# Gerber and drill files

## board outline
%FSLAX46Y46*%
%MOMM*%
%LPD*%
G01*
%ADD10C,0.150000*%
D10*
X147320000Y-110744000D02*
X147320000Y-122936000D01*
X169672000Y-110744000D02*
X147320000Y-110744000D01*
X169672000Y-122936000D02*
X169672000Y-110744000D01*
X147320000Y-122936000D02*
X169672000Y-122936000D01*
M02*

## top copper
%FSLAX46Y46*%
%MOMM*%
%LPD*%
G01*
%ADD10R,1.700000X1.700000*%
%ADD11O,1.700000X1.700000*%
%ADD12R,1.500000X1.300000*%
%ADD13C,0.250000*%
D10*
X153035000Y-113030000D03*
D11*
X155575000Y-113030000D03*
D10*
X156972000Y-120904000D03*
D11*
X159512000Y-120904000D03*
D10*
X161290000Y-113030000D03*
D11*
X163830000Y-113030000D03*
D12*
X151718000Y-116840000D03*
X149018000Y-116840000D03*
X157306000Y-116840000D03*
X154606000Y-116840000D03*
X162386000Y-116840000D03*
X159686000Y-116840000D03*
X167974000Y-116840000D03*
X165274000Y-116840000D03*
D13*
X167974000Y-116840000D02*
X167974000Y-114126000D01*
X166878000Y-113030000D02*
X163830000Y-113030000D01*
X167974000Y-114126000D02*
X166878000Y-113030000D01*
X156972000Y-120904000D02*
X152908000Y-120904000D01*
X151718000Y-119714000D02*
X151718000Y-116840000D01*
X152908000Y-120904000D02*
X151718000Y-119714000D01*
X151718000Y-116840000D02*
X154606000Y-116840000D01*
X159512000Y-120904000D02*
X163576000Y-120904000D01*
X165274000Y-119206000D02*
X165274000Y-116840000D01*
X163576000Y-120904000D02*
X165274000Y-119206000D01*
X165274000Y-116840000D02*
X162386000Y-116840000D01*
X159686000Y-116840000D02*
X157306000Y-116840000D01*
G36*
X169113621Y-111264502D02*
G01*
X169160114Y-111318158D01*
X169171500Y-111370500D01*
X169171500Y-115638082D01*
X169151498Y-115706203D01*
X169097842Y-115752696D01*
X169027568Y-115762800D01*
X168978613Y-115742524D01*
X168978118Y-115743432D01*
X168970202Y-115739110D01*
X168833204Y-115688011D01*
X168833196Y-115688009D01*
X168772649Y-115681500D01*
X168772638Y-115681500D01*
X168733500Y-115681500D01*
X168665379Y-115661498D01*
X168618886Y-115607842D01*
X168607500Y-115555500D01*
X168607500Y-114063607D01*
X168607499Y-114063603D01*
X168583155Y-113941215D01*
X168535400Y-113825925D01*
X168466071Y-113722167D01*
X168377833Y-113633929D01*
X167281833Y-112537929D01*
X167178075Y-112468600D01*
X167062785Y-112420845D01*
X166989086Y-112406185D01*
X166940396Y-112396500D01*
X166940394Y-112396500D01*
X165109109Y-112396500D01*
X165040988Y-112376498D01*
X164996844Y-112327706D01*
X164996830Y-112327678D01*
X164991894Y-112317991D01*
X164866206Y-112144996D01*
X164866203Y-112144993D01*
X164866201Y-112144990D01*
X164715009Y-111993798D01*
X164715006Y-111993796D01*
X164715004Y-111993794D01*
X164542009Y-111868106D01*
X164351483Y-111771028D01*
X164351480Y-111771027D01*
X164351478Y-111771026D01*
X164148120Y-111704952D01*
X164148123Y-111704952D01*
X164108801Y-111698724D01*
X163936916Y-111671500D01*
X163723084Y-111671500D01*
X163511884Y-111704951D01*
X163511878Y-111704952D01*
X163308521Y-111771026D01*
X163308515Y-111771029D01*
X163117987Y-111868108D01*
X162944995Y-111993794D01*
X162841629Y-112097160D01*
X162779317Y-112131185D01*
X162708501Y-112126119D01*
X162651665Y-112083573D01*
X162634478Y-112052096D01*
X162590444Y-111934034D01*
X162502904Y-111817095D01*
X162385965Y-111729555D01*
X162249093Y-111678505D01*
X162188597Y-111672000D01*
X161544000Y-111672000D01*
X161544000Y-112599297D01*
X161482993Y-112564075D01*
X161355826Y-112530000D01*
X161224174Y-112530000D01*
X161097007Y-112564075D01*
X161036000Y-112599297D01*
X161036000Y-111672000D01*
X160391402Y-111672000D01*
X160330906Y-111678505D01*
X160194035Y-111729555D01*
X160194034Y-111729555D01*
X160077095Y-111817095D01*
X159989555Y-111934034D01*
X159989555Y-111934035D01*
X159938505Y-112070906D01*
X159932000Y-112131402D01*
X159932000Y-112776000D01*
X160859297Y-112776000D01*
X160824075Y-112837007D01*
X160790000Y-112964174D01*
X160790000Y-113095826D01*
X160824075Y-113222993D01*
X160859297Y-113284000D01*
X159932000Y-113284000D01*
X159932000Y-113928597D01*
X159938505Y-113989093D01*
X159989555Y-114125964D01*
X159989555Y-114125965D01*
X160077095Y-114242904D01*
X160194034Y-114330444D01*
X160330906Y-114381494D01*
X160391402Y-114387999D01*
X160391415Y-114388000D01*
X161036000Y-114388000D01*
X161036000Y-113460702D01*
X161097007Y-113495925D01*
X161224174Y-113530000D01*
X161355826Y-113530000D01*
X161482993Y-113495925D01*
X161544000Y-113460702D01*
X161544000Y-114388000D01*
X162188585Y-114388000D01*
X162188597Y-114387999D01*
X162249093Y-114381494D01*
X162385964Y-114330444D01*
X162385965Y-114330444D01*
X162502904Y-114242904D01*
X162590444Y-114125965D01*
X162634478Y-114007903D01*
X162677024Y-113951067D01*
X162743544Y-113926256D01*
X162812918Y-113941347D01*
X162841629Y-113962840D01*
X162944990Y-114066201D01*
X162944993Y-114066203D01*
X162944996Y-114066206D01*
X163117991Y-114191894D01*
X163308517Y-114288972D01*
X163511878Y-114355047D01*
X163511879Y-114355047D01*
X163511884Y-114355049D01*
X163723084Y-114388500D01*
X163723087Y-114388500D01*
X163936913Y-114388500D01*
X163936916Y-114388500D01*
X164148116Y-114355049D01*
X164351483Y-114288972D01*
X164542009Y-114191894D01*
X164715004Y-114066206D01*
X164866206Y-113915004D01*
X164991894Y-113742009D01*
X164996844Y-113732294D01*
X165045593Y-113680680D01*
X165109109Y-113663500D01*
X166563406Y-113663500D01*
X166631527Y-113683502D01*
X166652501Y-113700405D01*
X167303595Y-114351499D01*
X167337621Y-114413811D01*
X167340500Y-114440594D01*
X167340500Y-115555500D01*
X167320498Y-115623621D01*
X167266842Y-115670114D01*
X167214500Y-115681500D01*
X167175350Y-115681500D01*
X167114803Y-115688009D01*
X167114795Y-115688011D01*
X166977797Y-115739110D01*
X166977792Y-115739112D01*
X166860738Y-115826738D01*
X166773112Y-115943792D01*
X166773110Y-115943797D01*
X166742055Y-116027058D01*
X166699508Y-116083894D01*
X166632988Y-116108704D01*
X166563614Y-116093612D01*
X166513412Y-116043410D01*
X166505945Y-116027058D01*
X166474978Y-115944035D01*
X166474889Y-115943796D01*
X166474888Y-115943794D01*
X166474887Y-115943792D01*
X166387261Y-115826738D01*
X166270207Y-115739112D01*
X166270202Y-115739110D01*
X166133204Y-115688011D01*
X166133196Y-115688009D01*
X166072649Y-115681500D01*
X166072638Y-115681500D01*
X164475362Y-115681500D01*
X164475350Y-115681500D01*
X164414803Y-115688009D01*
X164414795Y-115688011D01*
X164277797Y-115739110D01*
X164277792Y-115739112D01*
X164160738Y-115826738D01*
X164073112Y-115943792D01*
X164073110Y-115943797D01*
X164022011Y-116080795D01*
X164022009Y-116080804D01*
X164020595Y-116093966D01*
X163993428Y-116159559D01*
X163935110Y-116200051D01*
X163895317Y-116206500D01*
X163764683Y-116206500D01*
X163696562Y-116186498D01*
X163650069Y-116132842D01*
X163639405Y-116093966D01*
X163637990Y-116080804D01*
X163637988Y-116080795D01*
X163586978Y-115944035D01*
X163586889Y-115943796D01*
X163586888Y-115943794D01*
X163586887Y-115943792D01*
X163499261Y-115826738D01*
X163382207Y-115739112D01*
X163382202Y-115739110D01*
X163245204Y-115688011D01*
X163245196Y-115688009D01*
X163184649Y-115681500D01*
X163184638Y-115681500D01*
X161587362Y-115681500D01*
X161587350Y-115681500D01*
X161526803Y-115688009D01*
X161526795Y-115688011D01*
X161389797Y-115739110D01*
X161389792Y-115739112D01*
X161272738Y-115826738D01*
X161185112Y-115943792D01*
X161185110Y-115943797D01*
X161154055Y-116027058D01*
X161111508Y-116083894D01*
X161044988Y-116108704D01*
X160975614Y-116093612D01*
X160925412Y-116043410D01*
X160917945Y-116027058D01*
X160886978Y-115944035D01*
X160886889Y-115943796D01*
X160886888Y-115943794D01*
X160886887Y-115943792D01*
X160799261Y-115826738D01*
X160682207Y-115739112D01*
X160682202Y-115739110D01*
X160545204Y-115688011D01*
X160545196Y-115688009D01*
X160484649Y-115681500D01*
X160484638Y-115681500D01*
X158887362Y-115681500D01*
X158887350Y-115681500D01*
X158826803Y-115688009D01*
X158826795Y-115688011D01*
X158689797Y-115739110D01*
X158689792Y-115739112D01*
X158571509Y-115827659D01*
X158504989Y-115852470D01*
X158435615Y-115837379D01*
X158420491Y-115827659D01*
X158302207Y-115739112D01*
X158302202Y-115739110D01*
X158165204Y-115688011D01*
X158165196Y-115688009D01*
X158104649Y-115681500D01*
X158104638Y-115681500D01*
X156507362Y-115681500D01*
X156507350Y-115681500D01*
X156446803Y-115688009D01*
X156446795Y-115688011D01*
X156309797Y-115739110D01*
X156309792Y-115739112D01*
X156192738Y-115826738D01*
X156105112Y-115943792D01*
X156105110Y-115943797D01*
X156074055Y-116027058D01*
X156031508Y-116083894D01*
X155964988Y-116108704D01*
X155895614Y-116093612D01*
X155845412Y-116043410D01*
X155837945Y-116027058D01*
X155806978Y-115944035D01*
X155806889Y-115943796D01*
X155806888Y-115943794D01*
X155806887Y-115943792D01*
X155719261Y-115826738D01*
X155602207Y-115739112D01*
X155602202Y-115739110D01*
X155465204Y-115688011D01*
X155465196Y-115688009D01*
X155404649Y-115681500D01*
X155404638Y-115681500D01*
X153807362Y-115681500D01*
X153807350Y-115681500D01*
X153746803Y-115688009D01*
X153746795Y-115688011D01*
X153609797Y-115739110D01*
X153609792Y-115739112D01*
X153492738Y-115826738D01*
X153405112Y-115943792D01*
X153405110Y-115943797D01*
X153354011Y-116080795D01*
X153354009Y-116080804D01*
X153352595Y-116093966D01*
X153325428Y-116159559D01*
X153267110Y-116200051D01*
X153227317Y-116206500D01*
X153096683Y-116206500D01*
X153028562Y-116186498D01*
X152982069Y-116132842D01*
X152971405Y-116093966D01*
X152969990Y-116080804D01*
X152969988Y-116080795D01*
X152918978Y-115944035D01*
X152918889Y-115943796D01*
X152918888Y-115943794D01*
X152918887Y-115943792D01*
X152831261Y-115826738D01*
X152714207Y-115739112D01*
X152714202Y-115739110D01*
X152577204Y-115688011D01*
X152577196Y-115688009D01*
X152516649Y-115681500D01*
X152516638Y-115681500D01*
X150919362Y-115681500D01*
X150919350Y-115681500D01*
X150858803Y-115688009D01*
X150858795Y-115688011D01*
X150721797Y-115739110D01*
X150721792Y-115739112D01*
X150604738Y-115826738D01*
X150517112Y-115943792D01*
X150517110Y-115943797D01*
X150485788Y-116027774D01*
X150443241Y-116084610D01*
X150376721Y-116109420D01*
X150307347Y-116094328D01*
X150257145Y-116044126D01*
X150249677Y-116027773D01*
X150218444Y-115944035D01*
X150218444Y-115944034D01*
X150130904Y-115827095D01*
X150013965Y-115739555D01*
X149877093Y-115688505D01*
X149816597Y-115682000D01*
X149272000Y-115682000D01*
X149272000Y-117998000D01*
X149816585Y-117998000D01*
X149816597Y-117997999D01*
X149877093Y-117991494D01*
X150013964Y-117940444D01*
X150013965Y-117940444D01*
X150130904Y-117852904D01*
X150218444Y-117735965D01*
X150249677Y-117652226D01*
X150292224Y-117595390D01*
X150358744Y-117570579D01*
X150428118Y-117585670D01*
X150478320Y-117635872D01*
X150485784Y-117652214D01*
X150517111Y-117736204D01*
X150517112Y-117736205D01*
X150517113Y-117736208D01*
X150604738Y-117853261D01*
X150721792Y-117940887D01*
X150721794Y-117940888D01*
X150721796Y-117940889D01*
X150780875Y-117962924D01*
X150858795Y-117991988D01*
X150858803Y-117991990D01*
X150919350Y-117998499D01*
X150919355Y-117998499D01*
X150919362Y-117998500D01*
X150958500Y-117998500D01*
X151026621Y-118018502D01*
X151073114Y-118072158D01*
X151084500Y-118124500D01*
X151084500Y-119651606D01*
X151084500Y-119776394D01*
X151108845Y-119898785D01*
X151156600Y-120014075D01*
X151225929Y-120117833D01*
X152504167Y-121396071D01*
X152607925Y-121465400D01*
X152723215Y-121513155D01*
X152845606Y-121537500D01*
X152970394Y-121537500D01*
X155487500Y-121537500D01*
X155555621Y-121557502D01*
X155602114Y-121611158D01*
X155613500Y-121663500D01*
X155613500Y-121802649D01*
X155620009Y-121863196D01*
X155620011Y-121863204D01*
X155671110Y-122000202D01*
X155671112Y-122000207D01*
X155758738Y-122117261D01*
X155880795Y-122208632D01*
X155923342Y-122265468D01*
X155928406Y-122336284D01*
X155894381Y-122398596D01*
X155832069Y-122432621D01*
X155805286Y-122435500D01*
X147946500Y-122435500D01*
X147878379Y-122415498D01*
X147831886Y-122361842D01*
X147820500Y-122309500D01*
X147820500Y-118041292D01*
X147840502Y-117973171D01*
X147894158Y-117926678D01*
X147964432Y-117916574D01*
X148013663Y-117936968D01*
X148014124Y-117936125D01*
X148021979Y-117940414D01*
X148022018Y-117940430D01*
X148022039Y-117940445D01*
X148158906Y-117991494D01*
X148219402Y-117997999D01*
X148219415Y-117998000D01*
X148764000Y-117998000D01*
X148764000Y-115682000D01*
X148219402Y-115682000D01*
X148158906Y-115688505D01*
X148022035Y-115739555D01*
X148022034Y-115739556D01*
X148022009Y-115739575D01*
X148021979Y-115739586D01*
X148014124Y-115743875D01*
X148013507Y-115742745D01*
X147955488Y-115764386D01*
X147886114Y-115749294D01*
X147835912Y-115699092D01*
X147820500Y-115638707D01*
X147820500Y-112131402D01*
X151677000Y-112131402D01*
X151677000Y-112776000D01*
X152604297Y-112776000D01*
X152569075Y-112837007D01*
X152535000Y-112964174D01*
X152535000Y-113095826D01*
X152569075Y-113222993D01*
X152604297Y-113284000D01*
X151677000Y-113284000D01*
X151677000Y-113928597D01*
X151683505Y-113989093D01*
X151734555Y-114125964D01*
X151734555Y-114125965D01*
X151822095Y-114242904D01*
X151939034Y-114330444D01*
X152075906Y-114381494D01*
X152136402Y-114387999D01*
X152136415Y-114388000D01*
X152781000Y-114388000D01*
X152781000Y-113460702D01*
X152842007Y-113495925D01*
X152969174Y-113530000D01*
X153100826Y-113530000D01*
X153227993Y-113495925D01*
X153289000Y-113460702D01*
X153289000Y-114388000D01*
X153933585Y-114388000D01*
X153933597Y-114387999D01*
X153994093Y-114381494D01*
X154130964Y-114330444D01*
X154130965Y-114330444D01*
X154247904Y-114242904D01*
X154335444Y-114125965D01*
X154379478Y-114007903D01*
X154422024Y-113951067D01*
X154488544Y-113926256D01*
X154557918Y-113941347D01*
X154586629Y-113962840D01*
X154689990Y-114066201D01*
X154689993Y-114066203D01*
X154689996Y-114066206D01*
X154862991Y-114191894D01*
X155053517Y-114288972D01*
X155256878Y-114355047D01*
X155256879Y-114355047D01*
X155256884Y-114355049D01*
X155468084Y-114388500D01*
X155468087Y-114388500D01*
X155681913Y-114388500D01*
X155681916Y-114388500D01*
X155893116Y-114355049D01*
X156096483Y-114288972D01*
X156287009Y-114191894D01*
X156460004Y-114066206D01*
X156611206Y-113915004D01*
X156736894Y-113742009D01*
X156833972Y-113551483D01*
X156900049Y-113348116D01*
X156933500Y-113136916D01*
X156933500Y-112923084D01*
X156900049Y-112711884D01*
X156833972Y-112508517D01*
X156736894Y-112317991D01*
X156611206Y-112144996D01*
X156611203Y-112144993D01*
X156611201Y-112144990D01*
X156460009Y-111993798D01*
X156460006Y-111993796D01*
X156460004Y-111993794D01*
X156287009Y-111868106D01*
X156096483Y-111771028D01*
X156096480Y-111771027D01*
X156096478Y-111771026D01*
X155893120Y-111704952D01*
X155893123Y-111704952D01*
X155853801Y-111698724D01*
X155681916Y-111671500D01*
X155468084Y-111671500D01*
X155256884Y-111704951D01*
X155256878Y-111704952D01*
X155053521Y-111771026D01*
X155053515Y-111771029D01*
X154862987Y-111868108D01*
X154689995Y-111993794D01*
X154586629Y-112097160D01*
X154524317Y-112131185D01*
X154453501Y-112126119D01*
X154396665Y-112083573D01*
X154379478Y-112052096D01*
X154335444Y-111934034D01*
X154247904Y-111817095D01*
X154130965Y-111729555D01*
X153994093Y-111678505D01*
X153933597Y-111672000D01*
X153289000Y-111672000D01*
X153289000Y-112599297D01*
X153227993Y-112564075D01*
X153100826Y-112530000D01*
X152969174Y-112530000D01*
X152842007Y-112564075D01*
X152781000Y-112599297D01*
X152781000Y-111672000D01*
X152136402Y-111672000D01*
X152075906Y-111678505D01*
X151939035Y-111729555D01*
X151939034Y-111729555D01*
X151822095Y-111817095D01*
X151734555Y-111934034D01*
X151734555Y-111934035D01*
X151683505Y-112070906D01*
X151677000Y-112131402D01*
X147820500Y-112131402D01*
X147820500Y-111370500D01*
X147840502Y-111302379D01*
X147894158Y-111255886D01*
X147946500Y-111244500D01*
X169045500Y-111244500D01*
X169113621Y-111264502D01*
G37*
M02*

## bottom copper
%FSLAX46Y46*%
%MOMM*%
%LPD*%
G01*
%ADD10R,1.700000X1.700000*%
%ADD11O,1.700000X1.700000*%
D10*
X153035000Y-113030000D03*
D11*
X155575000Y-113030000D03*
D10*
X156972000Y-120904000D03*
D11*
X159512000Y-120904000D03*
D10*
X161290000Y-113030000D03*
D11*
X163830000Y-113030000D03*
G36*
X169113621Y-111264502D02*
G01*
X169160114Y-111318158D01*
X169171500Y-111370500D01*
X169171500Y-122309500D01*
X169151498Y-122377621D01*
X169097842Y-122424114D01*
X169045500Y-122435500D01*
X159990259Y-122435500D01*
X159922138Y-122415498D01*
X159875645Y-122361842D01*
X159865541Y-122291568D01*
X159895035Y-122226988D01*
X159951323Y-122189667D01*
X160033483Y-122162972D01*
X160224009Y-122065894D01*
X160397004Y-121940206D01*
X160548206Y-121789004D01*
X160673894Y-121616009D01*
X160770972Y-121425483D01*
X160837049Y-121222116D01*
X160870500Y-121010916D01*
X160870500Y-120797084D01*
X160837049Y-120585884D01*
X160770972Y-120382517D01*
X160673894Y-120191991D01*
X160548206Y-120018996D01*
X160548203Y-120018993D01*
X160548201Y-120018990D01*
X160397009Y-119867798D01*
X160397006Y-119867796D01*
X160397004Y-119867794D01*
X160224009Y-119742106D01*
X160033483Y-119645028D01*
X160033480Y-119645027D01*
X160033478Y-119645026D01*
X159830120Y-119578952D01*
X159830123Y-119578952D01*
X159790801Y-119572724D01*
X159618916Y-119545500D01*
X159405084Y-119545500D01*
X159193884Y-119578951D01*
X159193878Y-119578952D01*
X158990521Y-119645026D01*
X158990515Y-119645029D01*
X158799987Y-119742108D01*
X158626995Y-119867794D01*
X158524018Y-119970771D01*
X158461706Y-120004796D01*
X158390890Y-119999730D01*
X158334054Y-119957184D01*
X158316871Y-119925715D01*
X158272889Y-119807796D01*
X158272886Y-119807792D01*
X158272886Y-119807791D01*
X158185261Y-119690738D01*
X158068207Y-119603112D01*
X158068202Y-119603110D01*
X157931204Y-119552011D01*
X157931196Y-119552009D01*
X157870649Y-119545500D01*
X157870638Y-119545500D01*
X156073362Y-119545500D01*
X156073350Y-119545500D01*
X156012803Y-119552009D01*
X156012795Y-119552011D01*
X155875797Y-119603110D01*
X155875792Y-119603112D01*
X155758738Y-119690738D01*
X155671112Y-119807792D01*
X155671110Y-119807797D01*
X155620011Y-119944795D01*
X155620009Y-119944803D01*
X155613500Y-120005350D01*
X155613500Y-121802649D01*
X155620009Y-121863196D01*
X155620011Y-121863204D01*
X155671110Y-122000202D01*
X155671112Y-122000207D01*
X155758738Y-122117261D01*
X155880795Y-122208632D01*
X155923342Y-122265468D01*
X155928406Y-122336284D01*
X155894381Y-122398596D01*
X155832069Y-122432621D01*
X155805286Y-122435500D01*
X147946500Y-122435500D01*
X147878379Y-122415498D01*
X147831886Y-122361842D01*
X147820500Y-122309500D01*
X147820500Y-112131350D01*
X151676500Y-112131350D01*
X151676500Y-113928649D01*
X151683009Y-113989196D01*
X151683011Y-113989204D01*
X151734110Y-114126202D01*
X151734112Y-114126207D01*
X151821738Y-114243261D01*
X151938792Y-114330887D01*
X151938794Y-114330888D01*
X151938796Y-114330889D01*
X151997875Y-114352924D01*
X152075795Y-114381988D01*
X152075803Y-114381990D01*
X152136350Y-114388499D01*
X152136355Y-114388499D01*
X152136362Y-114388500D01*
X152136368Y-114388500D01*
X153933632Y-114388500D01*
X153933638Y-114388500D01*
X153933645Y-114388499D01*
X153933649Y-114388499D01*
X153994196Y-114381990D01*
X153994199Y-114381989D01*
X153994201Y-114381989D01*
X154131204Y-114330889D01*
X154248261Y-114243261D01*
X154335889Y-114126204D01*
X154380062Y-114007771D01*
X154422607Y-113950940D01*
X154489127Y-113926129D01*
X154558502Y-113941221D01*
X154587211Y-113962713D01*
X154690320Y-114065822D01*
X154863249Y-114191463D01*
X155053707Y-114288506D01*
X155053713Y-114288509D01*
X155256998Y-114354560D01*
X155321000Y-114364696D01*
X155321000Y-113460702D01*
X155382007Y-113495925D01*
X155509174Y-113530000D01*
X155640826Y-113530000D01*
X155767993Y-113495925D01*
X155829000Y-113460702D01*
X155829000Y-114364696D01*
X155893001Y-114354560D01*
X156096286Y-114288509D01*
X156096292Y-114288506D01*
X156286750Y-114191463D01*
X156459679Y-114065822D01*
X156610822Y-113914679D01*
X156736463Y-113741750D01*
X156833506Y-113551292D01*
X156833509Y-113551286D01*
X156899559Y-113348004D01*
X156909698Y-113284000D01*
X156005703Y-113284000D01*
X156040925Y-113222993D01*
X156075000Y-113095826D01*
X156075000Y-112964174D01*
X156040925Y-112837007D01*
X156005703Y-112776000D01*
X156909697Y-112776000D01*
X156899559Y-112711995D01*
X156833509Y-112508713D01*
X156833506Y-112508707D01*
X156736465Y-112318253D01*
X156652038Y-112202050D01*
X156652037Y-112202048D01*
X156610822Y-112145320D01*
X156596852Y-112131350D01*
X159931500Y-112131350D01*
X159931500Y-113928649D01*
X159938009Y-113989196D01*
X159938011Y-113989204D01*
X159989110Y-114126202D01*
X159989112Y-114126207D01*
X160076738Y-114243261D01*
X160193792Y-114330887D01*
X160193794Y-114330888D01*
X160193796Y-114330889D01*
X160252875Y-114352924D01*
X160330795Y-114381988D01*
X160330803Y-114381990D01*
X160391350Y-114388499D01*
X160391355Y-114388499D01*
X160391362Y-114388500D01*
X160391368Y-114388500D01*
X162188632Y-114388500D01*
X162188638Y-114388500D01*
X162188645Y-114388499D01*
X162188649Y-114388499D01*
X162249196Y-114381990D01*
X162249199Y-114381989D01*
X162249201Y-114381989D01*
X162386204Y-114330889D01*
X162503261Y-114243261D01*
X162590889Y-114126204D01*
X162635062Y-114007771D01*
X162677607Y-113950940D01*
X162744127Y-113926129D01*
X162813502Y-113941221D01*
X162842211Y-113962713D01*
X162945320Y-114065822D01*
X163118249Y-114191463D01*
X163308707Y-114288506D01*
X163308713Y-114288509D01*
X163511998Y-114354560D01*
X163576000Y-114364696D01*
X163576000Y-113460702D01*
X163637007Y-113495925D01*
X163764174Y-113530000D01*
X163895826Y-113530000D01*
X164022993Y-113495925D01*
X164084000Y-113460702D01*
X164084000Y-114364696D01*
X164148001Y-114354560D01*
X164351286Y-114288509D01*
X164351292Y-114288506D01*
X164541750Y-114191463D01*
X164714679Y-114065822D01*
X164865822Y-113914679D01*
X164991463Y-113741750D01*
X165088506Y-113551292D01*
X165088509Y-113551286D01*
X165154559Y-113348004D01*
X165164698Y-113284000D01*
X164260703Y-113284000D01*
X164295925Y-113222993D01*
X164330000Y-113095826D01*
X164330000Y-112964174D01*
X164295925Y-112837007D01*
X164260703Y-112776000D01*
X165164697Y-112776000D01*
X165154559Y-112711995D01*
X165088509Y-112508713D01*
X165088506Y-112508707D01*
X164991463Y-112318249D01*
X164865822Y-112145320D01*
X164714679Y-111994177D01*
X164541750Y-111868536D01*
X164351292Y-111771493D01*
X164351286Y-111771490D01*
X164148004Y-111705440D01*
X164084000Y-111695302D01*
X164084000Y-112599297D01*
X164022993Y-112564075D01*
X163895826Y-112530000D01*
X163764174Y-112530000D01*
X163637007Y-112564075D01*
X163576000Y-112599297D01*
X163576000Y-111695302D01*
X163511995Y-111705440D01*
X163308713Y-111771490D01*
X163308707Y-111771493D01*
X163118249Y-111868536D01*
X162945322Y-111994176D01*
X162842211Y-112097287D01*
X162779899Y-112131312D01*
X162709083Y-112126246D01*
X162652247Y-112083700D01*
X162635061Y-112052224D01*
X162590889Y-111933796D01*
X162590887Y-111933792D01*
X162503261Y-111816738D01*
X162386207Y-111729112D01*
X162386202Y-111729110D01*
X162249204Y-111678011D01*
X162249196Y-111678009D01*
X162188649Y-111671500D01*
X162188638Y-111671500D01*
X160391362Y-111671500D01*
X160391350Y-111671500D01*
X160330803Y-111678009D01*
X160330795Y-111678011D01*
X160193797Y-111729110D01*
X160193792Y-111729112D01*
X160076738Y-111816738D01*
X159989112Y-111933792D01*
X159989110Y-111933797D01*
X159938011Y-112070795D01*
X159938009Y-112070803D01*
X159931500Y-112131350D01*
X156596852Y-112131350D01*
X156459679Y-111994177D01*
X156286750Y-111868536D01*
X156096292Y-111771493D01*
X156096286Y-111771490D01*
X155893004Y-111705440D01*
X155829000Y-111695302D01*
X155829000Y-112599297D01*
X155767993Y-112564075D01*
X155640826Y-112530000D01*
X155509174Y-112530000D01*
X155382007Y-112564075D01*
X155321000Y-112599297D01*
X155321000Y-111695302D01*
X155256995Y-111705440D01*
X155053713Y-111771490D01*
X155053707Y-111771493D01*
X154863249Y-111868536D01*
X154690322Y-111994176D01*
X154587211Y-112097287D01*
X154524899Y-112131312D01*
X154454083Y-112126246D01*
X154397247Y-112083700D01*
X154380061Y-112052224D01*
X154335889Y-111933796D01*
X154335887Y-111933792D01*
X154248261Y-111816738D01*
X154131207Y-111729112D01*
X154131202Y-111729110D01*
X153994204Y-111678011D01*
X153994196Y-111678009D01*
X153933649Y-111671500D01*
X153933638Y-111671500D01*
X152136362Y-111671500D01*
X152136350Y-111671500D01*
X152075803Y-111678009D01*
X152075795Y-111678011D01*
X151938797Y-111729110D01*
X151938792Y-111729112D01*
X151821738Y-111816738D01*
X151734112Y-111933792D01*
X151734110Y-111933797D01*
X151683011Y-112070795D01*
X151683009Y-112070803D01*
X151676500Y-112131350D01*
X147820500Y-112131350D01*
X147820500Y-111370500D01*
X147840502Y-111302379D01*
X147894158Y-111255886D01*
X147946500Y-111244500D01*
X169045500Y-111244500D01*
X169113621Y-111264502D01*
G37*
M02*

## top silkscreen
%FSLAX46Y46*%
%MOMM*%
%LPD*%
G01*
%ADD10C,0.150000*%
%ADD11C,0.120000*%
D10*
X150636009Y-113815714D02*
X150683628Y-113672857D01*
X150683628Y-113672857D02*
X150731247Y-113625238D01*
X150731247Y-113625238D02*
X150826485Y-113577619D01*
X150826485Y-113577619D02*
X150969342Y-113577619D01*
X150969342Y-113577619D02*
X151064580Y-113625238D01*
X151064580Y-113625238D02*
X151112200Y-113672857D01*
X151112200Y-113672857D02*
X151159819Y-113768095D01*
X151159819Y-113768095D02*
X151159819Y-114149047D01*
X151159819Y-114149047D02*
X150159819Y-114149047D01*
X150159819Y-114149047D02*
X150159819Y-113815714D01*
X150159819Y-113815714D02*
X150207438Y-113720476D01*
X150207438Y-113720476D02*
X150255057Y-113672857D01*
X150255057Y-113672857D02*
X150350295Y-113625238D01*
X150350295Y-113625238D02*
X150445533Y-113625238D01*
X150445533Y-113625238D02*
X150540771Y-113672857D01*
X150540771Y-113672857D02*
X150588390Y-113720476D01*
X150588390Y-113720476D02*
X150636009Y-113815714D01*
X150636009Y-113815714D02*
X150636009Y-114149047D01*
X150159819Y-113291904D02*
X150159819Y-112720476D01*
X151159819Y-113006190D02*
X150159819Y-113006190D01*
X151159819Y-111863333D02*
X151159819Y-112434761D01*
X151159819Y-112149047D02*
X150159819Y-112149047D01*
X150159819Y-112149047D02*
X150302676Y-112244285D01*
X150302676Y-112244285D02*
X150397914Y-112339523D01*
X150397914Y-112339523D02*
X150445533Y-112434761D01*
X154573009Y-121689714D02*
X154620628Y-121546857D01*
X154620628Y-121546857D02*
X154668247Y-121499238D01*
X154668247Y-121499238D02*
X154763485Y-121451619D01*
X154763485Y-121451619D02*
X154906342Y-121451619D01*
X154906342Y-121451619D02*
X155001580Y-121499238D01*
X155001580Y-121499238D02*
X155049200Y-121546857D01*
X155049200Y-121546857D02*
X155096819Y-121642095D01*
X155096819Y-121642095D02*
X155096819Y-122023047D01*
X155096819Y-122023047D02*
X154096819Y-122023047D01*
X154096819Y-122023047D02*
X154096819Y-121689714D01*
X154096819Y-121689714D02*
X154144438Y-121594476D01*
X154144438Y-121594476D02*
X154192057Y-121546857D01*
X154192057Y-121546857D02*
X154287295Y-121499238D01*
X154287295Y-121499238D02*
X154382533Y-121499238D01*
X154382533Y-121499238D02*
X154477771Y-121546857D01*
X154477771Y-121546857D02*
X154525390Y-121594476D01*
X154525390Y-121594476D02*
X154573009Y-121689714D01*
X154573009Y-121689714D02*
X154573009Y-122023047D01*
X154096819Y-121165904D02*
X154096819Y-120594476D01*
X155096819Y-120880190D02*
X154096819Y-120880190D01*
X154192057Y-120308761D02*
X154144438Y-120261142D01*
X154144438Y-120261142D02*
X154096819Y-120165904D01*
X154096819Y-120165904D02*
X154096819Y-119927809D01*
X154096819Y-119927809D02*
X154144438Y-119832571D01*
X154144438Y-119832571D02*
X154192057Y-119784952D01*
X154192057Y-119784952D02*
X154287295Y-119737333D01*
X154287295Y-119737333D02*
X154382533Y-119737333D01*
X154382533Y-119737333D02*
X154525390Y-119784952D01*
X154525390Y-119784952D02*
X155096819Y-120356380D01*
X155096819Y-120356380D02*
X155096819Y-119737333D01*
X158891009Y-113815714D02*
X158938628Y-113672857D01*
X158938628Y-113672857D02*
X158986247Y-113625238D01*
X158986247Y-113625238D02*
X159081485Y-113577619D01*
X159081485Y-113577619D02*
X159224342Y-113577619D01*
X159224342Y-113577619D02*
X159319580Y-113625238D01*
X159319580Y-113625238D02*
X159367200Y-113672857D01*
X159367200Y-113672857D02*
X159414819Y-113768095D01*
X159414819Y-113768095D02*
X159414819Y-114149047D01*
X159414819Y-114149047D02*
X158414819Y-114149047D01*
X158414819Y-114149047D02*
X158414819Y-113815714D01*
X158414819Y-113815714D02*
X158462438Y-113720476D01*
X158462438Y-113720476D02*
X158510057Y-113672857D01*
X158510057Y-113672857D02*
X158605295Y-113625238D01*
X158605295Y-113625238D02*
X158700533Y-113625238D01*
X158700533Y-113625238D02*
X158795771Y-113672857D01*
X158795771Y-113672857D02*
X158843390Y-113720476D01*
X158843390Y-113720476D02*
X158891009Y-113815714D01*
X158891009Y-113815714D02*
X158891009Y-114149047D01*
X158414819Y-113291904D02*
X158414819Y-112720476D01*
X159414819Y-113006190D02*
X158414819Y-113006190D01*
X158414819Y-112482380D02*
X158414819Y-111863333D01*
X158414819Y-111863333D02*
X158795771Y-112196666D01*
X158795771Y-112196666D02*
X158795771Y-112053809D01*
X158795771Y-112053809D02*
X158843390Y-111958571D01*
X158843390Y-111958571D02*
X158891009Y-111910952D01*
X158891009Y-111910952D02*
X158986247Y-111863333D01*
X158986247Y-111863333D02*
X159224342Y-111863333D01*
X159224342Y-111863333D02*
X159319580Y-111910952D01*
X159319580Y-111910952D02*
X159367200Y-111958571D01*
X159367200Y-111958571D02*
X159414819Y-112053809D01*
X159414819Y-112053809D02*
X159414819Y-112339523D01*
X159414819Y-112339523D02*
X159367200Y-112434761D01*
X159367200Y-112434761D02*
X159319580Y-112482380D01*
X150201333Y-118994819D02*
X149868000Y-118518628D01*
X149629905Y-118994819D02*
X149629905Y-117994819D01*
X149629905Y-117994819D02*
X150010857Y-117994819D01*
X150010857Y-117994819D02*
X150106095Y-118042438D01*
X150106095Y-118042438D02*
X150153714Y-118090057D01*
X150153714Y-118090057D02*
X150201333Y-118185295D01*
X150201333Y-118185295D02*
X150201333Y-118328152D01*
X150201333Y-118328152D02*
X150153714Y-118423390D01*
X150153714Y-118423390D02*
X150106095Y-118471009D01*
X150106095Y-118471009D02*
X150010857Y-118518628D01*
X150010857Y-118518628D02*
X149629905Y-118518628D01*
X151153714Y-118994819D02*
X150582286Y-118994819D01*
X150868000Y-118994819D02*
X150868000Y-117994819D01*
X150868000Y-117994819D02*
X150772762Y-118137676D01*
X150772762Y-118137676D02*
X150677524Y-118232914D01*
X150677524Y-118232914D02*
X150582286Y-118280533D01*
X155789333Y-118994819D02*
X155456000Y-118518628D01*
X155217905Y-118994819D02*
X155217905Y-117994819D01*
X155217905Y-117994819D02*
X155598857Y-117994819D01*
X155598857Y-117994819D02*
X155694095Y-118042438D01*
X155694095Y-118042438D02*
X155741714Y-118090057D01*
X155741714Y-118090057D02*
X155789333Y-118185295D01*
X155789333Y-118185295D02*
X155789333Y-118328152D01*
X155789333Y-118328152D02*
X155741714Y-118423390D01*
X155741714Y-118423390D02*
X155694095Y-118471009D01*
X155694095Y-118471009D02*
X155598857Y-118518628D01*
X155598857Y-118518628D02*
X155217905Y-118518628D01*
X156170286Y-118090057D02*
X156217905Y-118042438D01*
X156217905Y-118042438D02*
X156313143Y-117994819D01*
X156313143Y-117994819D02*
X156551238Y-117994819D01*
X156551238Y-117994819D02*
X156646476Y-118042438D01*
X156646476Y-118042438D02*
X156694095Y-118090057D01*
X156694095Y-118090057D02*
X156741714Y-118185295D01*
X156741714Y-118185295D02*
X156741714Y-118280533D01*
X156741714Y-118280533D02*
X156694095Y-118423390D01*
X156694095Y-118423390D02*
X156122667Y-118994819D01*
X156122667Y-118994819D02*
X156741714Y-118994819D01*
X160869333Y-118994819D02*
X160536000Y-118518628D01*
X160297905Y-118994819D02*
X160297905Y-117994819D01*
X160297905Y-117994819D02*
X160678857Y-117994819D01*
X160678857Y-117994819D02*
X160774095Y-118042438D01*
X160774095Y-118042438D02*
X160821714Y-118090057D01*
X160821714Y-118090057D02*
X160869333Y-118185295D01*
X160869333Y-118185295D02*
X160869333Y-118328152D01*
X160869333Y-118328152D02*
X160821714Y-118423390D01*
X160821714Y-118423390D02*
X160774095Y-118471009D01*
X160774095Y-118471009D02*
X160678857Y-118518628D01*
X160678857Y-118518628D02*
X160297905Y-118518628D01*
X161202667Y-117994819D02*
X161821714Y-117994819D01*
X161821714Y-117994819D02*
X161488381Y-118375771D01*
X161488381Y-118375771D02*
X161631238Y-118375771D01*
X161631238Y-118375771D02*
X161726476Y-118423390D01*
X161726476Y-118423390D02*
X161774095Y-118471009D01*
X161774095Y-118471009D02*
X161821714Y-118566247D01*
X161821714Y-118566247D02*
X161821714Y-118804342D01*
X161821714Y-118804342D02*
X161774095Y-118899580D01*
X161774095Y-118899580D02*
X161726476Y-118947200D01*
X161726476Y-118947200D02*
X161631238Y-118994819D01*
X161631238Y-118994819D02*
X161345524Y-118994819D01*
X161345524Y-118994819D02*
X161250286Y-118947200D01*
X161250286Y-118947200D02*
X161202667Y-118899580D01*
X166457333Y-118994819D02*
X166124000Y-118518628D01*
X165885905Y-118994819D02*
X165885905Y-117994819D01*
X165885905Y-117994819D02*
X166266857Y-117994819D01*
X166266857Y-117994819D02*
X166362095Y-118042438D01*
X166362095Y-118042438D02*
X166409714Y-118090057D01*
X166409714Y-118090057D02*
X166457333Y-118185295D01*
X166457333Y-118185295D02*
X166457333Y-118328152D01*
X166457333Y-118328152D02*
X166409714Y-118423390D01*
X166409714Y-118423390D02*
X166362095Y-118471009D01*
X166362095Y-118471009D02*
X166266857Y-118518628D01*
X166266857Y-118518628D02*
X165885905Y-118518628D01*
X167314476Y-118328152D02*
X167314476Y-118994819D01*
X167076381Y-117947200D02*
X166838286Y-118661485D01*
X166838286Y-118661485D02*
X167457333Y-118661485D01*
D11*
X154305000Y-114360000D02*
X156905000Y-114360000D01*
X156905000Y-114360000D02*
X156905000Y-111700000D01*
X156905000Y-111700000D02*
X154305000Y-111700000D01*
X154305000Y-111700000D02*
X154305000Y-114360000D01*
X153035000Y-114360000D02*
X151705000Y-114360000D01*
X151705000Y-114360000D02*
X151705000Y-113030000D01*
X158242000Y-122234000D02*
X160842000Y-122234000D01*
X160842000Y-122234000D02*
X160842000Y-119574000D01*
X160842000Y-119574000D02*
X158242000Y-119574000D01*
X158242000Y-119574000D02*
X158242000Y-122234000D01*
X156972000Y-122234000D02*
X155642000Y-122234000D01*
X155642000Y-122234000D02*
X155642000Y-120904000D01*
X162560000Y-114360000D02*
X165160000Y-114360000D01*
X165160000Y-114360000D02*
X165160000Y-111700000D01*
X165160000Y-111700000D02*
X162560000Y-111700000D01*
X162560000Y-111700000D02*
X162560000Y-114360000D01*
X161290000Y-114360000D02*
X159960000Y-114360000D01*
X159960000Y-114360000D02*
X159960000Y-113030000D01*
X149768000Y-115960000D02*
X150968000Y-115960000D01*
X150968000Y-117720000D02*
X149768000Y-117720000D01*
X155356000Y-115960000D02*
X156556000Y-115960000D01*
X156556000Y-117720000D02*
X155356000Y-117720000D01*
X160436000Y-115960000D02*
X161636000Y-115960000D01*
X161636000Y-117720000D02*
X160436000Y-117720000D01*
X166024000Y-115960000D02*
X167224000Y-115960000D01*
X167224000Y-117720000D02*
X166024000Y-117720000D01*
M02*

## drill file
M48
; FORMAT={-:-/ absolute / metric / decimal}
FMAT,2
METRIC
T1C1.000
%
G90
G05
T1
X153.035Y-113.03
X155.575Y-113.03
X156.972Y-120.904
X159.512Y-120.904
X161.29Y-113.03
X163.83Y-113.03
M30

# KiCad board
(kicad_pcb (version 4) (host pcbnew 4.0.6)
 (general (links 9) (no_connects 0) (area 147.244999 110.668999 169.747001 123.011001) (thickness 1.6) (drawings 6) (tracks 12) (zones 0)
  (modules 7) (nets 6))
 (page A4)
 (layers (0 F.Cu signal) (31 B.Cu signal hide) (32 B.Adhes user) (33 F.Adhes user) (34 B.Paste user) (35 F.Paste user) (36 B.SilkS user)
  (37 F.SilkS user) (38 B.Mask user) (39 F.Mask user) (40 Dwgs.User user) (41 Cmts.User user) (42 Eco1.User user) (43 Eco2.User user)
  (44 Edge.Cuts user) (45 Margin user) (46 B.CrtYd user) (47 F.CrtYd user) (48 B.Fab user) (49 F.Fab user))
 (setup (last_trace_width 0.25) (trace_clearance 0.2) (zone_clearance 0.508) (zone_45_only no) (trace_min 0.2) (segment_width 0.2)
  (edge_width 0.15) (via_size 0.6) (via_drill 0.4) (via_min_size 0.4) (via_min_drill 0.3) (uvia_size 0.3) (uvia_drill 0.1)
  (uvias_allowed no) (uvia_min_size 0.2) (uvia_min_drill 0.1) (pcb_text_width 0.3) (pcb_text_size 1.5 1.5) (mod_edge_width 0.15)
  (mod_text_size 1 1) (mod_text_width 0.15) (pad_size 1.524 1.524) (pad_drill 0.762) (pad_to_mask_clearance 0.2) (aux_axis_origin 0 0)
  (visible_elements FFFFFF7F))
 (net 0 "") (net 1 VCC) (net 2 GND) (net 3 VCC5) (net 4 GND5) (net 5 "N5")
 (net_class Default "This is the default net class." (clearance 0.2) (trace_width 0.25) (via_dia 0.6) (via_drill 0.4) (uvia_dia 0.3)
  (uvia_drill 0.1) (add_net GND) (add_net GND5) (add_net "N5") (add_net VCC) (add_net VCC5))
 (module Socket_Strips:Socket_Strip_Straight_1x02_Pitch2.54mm (layer F.Cu) (at 153.035 113.03 90)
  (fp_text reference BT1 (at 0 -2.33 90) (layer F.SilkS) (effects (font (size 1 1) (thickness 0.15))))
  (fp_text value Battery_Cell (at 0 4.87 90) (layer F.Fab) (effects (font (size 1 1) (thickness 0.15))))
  (fp_line (start -1.33 1.27) (end -1.33 3.87) (layer F.SilkS) (width 0.12))
  (fp_line (start -1.33 3.87) (end 1.33 3.87) (layer F.SilkS) (width 0.12))
  (fp_line (start 1.33 3.87) (end 1.33 1.27) (layer F.SilkS) (width 0.12))
  (fp_line (start 1.33 1.27) (end -1.33 1.27) (layer F.SilkS) (width 0.12))
  (fp_line (start -1.33 0) (end -1.33 -1.33) (layer F.SilkS) (width 0.12))
  (fp_line (start -1.33 -1.33) (end 0 -1.33) (layer F.SilkS) (width 0.12))
  (pad 1 thru_hole rect (at 0 0 90) (size 1.7 1.7) (drill 1) (layers *.Cu *.Mask) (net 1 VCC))
  (pad 2 thru_hole oval (at 0 2.54 90) (size 1.7 1.7) (drill 1) (layers *.Cu *.Mask) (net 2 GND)))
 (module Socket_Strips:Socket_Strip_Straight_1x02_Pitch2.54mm (layer F.Cu) (at 156.972 120.904 90)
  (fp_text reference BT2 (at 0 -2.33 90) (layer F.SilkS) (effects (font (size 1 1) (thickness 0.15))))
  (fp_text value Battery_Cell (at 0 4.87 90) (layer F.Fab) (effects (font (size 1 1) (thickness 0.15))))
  (fp_line (start -1.33 1.27) (end -1.33 3.87) (layer F.SilkS) (width 0.12))
  (fp_line (start -1.33 3.87) (end 1.33 3.87) (layer F.SilkS) (width 0.12))
  (fp_line (start 1.33 3.87) (end 1.33 1.27) (layer F.SilkS) (width 0.12))
  (fp_line (start 1.33 1.27) (end -1.33 1.27) (layer F.SilkS) (width 0.12))
  (fp_line (start -1.33 0) (end -1.33 -1.33) (layer F.SilkS) (width 0.12))
  (fp_line (start -1.33 -1.33) (end 0 -1.33) (layer F.SilkS) (width 0.12))
  (pad 1 thru_hole rect (at 0 0 90) (size 1.7 1.7) (drill 1) (layers *.Cu *.Mask) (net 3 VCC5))
  (pad 2 thru_hole oval (at 0 2.54 90) (size 1.7 1.7) (drill 1) (layers *.Cu *.Mask) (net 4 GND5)))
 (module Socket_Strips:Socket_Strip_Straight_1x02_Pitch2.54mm (layer F.Cu) (at 161.29 113.03 90)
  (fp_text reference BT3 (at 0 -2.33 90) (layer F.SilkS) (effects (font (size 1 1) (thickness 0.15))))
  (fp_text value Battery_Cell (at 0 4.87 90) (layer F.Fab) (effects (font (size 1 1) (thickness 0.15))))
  (fp_line (start -1.33 1.27) (end -1.33 3.87) (layer F.SilkS) (width 0.12))
  (fp_line (start -1.33 3.87) (end 1.33 3.87) (layer F.SilkS) (width 0.12))
  (fp_line (start 1.33 3.87) (end 1.33 1.27) (layer F.SilkS) (width 0.12))
  (fp_line (start 1.33 1.27) (end -1.33 1.27) (layer F.SilkS) (width 0.12))
  (fp_line (start -1.33 0) (end -1.33 -1.33) (layer F.SilkS) (width 0.12))
  (fp_line (start -1.33 -1.33) (end 0 -1.33) (layer F.SilkS) (width 0.12))
  (pad 1 thru_hole rect (at 0 0 90) (size 1.7 1.7) (drill 1) (layers *.Cu *.Mask) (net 1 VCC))
  (pad 2 thru_hole oval (at 0 2.54 90) (size 1.7 1.7) (drill 1) (layers *.Cu *.Mask) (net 2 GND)))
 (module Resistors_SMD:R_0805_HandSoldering (layer F.Cu) (at 150.368 116.84 180)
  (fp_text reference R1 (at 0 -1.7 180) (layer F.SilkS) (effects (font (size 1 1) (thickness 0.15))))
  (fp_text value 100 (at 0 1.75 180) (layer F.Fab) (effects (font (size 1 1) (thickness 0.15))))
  (fp_line (start 0.6 0.88) (end -0.6 0.88) (layer F.SilkS) (width 0.12))
  (fp_line (start -0.6 -0.88) (end 0.6 -0.88) (layer F.SilkS) (width 0.12))
  (pad 1 smd rect (at -1.35 0 180) (size 1.5 1.3) (layers F.Cu F.Paste F.Mask) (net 3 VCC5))
  (pad 2 smd rect (at 1.35 0 180) (size 1.5 1.3) (layers F.Cu F.Paste F.Mask) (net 1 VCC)))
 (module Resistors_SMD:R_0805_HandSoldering (layer F.Cu) (at 155.956 116.84 180)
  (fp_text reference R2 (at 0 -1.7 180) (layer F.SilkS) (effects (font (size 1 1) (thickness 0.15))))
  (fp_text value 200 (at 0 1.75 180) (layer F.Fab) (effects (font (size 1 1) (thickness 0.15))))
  (fp_line (start 0.6 0.88) (end -0.6 0.88) (layer F.SilkS) (width 0.12))
  (fp_line (start -0.6 -0.88) (end 0.6 -0.88) (layer F.SilkS) (width 0.12))
  (pad 1 smd rect (at -1.35 0 180) (size 1.5 1.3) (layers F.Cu F.Paste F.Mask) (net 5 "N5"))
  (pad 2 smd rect (at 1.35 0 180) (size 1.5 1.3) (layers F.Cu F.Paste F.Mask) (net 3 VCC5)))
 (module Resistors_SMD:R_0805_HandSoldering (layer F.Cu) (at 161.036 116.84 180)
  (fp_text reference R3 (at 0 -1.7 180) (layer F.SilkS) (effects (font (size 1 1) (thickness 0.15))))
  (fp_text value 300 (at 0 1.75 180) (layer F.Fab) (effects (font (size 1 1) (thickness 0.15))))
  (fp_line (start 0.6 0.88) (end -0.6 0.88) (layer F.SilkS) (width 0.12))
  (fp_line (start -0.6 -0.88) (end 0.6 -0.88) (layer F.SilkS) (width 0.12))
  (pad 1 smd rect (at -1.35 0 180) (size 1.5 1.3) (layers F.Cu F.Paste F.Mask) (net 4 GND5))
  (pad 2 smd rect (at 1.35 0 180) (size 1.5 1.3) (layers F.Cu F.Paste F.Mask) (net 5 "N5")))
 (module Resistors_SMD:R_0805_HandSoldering (layer F.Cu) (at 166.624 116.84 180)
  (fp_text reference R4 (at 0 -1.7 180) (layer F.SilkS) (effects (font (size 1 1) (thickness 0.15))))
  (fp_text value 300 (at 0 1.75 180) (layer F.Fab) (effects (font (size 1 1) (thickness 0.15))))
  (fp_line (start 0.6 0.88) (end -0.6 0.88) (layer F.SilkS) (width 0.12))
  (fp_line (start -0.6 -0.88) (end 0.6 -0.88) (layer F.SilkS) (width 0.12))
  (pad 1 smd rect (at -1.35 0 180) (size 1.5 1.3) (layers F.Cu F.Paste F.Mask) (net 2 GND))
  (pad 2 smd rect (at 1.35 0 180) (size 1.5 1.3) (layers F.Cu F.Paste F.Mask) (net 4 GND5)))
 (gr_line (start 147.32 110.744) (end 147.32 122.936) (angle 90) (layer Edge.Cuts) (width 0.15))
 (gr_line (start 169.672 110.744) (end 147.32 110.744) (angle 90) (layer Edge.Cuts) (width 0.15))
 (gr_line (start 169.672 122.936) (end 169.672 110.744) (angle 90) (layer Edge.Cuts) (width 0.15))
 (gr_line (start 147.32 122.936) (end 169.672 122.936) (angle 90) (layer Edge.Cuts) (width 0.15))
 (segment (start 167.974 116.84) (end 167.974 114.126) (width 0.25) (layer F.Cu) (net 2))
 (segment (start 166.878 113.03) (end 163.83 113.03) (width 0.25) (layer F.Cu) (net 2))
 (segment (start 167.974 114.126) (end 166.878 113.03) (width 0.25) (layer F.Cu) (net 2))
 (segment (start 156.972 120.904) (end 152.908 120.904) (width 0.25) (layer F.Cu) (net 3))
 (segment (start 151.718 119.714) (end 151.718 116.84) (width 0.25) (layer F.Cu) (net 3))
 (segment (start 152.908 120.904) (end 151.718 119.714) (width 0.25) (layer F.Cu) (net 3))
 (segment (start 151.718 116.84) (end 154.606 116.84) (width 0.25) (layer F.Cu) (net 3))
 (segment (start 159.512 120.904) (end 163.576 120.904) (width 0.25) (layer F.Cu) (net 4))
 (segment (start 165.274 119.206) (end 165.274 116.84) (width 0.25) (layer F.Cu) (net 4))
 (segment (start 163.576 120.904) (end 165.274 119.206) (width 0.25) (layer F.Cu) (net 4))
 (segment (start 165.274 116.84) (end 162.386 116.84) (width 0.25) (layer F.Cu) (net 4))
 (segment (start 159.686 116.84) (end 157.306 116.84) (width 0.25) (layer F.Cu) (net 5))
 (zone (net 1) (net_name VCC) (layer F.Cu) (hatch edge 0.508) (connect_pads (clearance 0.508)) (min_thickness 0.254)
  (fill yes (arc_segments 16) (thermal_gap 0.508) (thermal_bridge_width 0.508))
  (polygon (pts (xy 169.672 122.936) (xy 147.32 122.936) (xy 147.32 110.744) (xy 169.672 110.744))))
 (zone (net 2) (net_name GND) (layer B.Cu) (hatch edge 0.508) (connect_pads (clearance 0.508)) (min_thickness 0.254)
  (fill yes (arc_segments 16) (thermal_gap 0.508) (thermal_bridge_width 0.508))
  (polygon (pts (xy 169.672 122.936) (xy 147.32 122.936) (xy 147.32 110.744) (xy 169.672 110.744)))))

